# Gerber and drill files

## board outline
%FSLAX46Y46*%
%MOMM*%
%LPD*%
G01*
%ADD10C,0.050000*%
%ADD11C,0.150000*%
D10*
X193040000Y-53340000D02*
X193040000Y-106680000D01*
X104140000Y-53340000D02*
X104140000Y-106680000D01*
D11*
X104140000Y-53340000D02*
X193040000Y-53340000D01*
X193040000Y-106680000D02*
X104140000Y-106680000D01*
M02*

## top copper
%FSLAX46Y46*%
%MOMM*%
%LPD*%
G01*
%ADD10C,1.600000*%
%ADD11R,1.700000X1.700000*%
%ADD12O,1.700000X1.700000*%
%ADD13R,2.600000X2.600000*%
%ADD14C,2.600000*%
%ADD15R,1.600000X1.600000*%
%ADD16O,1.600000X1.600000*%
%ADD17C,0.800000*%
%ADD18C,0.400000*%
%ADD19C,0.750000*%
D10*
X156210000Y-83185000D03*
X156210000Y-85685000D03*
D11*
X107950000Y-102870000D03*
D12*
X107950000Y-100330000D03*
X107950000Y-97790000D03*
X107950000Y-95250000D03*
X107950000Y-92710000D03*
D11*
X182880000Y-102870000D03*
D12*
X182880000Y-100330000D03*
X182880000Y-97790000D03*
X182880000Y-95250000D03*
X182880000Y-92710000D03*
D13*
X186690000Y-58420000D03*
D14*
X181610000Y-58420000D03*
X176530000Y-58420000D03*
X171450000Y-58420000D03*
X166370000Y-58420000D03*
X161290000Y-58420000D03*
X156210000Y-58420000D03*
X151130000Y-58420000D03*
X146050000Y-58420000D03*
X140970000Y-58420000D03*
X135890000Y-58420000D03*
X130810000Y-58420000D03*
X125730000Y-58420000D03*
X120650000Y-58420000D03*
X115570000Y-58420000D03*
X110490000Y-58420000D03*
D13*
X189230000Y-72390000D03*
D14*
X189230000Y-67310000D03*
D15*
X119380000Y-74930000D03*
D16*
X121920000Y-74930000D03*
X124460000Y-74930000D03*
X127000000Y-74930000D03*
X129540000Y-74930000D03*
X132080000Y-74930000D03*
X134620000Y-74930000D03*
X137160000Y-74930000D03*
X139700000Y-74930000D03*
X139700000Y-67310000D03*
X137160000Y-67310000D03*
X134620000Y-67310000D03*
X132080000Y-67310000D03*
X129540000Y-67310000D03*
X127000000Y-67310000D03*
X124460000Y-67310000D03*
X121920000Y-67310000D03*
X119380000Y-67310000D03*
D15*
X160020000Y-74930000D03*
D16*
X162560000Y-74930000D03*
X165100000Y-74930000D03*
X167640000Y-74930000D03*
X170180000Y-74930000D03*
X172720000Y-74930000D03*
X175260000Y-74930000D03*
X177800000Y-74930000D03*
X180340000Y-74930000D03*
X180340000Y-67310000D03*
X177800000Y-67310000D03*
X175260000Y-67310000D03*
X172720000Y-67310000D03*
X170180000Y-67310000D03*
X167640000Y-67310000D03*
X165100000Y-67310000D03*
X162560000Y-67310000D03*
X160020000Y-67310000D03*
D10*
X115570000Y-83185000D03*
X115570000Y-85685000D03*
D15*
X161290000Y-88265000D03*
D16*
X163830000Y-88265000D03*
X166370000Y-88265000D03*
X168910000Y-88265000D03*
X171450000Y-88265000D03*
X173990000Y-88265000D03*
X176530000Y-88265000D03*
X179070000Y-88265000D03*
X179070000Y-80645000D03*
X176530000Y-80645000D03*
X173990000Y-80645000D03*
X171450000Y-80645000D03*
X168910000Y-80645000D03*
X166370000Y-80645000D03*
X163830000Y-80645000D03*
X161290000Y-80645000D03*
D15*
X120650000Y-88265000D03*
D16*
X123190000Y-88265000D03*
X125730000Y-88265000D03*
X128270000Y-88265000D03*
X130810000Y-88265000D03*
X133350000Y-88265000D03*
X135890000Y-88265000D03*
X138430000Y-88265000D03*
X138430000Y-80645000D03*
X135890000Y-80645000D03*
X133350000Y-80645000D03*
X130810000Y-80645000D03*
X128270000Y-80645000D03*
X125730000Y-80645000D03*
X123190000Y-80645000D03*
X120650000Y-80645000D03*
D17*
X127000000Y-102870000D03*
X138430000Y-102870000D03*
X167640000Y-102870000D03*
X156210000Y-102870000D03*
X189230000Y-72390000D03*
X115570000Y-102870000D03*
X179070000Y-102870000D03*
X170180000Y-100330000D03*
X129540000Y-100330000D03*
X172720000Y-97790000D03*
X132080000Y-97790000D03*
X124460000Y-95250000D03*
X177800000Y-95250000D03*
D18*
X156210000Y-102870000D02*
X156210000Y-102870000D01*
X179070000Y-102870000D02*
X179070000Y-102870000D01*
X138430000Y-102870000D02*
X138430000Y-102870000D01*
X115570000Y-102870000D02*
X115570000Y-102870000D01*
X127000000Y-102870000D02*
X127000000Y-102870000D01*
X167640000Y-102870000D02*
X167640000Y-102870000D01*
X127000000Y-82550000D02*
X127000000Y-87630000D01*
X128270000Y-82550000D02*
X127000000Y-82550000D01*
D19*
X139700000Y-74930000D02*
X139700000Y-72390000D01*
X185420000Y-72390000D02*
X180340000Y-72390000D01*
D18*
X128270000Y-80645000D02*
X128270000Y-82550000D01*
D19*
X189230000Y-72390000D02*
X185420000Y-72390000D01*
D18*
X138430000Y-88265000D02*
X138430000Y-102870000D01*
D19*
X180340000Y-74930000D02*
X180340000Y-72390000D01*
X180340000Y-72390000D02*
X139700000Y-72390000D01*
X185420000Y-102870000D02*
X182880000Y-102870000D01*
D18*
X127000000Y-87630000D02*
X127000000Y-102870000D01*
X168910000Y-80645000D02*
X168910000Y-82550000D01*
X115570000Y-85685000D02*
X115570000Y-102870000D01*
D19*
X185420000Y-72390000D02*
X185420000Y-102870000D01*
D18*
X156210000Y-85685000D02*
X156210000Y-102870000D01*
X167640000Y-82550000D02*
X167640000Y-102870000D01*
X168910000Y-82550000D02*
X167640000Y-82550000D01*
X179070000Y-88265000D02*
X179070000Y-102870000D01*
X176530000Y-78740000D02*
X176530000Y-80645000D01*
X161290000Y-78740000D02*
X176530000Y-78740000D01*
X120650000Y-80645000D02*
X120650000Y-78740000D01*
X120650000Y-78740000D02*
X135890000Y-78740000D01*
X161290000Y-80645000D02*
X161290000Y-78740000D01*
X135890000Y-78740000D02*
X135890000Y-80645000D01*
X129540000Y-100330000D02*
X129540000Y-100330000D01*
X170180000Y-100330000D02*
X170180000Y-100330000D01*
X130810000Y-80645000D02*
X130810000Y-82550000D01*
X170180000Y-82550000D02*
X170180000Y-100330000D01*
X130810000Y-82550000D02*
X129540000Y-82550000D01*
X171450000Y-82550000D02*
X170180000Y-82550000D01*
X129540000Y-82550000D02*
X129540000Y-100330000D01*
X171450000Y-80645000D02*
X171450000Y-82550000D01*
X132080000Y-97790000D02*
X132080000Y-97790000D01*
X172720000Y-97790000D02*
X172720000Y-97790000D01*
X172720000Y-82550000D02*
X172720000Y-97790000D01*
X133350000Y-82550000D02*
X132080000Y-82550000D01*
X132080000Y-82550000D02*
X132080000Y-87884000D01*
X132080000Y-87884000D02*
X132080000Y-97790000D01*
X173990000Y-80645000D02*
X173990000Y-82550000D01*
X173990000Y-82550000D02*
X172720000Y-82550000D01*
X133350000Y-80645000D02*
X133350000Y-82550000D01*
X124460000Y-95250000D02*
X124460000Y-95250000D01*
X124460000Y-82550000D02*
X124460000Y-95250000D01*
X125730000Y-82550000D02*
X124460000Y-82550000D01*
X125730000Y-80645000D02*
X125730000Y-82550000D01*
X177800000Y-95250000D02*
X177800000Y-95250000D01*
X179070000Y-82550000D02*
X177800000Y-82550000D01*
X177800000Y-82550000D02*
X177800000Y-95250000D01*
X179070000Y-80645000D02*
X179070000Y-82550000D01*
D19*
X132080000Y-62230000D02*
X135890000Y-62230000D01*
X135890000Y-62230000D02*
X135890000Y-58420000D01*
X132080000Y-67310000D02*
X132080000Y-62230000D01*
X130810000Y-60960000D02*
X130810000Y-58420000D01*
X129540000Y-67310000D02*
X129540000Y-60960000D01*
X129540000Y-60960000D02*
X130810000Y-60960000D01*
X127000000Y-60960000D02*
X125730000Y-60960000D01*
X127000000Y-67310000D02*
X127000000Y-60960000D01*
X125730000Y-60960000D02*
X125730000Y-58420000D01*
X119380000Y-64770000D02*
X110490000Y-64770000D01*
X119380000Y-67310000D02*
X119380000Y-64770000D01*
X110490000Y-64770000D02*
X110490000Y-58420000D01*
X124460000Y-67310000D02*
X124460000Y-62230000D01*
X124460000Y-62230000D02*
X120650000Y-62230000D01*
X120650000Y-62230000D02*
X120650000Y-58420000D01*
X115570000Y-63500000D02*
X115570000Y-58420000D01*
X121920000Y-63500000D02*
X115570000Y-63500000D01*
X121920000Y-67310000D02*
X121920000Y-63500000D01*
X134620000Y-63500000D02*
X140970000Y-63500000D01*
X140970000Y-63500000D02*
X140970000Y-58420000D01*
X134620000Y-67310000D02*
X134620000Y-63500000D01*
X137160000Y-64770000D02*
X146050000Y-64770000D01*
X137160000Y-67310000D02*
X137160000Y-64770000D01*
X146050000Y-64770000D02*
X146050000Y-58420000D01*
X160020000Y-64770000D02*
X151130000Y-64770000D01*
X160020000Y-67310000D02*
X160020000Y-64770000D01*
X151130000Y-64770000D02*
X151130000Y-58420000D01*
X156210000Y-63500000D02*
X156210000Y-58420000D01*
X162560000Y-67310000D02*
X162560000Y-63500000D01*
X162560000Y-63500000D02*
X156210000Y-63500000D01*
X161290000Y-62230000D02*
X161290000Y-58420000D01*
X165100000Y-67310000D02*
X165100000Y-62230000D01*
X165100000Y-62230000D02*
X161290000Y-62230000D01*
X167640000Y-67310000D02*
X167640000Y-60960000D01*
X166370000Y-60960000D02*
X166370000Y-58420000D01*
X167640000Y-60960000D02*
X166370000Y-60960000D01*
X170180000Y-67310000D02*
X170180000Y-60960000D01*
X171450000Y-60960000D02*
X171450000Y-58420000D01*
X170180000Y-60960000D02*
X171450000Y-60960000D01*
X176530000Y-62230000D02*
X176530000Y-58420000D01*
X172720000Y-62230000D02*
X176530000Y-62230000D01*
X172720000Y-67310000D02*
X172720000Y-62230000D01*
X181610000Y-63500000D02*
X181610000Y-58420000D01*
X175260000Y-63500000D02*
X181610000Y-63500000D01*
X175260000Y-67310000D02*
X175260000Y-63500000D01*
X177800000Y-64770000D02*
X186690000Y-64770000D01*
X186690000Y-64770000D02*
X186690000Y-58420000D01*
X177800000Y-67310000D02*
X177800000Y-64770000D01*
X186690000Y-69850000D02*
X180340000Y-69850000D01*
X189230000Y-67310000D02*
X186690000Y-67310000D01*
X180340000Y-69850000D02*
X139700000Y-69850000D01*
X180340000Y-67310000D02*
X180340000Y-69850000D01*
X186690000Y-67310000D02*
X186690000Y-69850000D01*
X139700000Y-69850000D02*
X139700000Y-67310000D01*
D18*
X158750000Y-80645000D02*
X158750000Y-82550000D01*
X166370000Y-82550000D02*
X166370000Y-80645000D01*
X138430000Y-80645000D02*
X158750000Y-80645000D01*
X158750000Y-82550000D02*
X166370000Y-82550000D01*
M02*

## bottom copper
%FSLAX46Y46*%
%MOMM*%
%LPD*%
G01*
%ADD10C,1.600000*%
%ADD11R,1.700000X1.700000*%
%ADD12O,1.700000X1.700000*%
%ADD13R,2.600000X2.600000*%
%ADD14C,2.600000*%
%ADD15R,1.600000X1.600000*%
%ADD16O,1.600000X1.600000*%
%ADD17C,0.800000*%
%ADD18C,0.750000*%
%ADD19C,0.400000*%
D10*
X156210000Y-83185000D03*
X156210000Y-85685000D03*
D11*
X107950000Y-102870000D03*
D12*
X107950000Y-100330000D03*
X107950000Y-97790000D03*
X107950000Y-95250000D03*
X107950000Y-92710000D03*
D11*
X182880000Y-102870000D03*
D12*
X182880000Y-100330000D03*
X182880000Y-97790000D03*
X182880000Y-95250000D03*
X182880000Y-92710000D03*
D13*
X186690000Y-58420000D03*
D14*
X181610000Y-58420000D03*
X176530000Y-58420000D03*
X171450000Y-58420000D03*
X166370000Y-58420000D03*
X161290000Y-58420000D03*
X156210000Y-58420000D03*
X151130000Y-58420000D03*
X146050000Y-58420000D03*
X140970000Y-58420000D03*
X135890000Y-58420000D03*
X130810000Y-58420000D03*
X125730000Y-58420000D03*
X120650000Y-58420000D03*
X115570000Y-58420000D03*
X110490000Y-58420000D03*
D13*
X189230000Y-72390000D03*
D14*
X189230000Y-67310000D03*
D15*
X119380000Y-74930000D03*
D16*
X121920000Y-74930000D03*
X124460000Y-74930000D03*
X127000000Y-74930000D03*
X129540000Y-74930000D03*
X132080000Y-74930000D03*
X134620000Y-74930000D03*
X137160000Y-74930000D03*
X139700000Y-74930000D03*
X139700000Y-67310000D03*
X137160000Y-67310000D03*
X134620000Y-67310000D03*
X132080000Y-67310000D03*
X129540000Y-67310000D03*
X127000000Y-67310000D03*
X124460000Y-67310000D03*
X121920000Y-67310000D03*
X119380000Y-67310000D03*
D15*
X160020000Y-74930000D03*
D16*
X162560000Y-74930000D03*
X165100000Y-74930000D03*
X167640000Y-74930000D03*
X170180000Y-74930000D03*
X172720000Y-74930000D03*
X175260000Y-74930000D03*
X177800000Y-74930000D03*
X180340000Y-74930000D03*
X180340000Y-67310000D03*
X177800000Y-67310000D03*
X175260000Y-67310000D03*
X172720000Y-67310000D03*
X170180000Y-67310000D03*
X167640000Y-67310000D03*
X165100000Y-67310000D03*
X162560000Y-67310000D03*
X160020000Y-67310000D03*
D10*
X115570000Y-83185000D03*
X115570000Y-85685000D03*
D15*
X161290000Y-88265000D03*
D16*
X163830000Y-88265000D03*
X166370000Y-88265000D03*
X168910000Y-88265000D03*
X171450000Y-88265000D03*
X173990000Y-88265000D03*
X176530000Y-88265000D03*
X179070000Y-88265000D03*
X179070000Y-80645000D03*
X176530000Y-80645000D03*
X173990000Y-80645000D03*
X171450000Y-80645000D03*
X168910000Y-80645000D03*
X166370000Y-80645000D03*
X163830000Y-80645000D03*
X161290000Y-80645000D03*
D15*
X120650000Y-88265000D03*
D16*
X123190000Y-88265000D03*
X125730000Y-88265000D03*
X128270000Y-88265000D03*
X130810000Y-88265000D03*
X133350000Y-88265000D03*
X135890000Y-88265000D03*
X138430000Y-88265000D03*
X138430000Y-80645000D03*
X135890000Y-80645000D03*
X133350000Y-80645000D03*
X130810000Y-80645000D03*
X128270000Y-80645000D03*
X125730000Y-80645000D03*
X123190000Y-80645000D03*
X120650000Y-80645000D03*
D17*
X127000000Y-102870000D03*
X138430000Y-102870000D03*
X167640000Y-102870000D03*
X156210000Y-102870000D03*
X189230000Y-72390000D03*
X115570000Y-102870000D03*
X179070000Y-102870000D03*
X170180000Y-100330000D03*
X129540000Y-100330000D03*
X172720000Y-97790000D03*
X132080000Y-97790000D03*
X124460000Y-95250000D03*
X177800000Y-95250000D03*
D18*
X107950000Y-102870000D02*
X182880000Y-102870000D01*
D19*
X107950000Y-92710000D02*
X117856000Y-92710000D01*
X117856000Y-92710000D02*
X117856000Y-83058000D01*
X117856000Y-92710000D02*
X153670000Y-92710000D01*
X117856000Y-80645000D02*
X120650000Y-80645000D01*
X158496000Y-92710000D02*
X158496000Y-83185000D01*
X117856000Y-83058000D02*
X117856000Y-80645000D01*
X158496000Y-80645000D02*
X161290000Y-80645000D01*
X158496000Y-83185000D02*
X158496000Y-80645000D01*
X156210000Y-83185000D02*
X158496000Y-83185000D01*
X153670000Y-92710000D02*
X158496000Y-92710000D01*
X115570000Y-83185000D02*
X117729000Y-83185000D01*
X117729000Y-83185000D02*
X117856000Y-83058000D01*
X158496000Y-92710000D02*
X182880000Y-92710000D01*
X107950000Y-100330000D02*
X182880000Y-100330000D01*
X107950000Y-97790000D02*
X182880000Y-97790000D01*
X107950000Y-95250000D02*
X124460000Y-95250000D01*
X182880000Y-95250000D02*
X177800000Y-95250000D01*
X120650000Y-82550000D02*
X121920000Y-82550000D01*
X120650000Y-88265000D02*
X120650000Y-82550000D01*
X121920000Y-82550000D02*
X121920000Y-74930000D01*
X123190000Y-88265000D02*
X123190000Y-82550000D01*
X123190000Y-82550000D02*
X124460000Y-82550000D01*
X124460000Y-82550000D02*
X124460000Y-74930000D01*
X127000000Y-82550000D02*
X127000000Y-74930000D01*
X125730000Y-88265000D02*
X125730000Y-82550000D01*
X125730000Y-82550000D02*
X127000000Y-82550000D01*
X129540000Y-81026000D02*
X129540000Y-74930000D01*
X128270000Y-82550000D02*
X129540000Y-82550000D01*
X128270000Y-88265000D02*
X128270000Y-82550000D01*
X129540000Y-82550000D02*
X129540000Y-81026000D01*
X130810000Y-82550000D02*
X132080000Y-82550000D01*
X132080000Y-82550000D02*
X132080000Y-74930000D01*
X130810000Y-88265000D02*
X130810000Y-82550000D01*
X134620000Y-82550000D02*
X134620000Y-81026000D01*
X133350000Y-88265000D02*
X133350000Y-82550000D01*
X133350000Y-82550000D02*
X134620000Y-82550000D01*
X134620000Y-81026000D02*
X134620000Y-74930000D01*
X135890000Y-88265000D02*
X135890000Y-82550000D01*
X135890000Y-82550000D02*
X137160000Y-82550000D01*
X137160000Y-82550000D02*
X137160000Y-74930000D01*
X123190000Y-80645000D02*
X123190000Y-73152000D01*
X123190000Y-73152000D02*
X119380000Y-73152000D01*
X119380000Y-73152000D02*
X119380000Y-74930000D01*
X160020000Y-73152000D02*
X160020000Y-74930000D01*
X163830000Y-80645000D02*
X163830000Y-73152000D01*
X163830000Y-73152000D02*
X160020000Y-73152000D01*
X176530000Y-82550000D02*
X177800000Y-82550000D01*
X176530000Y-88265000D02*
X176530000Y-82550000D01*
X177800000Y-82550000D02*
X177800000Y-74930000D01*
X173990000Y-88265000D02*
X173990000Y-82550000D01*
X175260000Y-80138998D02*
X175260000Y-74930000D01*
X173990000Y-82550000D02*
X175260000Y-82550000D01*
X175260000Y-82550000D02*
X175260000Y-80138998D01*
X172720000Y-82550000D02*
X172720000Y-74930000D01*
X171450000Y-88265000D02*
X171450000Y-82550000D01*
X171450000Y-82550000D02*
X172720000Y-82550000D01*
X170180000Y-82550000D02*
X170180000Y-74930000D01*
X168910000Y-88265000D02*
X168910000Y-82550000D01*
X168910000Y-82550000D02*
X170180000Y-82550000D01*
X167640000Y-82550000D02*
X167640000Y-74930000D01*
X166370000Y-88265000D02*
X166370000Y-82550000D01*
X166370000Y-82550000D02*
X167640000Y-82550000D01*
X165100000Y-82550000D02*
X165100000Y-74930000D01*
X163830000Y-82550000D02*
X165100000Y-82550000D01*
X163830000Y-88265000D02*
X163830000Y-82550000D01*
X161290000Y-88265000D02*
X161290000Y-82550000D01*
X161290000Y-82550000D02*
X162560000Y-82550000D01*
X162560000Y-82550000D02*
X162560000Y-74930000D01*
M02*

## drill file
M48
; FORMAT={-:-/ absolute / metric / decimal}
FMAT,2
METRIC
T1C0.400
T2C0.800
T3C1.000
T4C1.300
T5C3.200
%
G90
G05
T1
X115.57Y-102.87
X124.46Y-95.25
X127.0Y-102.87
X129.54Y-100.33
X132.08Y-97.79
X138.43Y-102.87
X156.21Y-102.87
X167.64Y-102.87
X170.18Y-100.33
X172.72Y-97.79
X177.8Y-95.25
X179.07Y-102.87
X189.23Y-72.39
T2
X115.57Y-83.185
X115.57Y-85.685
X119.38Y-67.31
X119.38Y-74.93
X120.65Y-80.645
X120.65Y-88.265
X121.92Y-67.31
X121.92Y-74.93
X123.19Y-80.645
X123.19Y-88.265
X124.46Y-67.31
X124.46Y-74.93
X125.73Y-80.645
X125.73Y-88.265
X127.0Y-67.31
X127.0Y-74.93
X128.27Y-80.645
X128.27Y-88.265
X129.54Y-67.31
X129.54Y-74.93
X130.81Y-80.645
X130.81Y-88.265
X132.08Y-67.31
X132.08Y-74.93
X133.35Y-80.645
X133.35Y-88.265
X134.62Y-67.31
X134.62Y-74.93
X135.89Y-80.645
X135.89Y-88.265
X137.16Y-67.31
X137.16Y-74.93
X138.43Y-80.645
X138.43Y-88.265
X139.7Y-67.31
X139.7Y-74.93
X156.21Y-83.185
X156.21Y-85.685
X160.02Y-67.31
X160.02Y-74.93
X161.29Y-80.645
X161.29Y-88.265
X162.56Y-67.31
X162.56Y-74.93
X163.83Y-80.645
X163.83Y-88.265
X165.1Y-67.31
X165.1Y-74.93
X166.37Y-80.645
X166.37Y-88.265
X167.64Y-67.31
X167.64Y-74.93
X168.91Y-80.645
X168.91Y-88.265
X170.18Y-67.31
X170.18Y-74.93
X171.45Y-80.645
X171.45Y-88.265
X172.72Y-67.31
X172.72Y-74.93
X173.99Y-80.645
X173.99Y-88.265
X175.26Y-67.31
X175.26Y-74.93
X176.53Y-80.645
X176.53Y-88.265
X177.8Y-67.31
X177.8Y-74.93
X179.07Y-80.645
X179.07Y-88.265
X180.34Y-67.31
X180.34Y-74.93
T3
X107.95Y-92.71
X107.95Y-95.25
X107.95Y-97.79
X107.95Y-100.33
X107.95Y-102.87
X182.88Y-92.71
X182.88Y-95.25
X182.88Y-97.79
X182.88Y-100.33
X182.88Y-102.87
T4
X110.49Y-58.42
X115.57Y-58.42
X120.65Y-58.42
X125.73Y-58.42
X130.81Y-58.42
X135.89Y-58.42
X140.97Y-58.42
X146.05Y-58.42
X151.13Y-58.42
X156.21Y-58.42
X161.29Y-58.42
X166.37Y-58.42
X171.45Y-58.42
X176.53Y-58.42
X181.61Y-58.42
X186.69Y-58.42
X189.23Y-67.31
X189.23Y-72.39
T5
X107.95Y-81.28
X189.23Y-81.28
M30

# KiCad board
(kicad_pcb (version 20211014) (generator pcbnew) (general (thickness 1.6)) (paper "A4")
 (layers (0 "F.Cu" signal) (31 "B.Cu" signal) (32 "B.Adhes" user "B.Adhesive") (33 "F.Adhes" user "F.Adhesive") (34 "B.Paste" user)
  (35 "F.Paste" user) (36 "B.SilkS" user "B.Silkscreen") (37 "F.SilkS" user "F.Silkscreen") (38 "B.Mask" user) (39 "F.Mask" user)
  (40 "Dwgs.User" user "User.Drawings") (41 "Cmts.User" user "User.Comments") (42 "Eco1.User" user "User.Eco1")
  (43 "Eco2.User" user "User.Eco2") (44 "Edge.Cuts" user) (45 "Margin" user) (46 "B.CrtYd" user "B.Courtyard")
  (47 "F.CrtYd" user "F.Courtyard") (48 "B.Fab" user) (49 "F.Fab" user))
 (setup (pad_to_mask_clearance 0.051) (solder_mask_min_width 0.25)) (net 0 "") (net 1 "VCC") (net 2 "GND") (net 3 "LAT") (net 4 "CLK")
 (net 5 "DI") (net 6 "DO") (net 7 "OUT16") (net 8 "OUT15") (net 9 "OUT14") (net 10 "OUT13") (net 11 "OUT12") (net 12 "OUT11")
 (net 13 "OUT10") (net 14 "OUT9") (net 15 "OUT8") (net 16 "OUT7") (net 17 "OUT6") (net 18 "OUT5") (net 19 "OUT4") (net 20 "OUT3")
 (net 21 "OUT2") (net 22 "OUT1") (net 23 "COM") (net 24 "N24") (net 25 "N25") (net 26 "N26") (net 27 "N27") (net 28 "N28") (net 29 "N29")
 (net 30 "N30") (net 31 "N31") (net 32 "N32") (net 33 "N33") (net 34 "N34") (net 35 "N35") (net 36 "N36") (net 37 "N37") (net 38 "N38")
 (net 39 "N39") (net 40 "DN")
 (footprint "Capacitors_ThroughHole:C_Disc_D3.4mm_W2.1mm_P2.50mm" (layer "F.Cu") (at 156.21 83.185 -90)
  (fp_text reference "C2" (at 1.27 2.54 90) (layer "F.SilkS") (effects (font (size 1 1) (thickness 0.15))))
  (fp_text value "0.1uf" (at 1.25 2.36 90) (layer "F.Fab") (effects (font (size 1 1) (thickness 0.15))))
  (pad "1" thru_hole circle locked (at 0 0 270) (size 1.6 1.6) (drill 0.8) (layers *.Cu *.Mask) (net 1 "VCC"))
  (pad "2" thru_hole circle locked (at 2.5 0 270) (size 1.6 1.6) (drill 0.8) (layers *.Cu *.Mask) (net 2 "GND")))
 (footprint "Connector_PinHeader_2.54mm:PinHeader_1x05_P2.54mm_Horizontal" (layer "F.Cu") (at 107.95 102.87 180)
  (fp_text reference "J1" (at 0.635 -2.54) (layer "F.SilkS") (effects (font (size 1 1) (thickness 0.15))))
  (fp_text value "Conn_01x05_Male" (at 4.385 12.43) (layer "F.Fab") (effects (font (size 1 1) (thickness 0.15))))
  (pad "1" thru_hole rect locked (at 0 0 180) (size 1.7 1.7) (drill 1) (layers *.Cu *.Mask) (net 2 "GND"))
  (pad "2" thru_hole oval locked (at 0 2.54 180) (size 1.7 1.7) (drill 1) (layers *.Cu *.Mask) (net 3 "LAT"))
  (pad "3" thru_hole oval locked (at 0 5.08 180) (size 1.7 1.7) (drill 1) (layers *.Cu *.Mask) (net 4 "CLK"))
  (pad "4" thru_hole oval locked (at 0 7.62 180) (size 1.7 1.7) (drill 1) (layers *.Cu *.Mask) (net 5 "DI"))
  (pad "5" thru_hole oval locked (at 0 10.16 180) (size 1.7 1.7) (drill 1) (layers *.Cu *.Mask) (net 1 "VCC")))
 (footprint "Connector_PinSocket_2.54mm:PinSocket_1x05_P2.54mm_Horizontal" (layer "F.Cu") (at 182.88 102.87 180)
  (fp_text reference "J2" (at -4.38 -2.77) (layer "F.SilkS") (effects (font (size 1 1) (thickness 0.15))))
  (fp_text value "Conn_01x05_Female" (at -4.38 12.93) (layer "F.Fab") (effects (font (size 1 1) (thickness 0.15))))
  (pad "1" thru_hole rect locked (at 0 0 180) (size 1.7 1.7) (drill 1) (layers *.Cu *.Mask) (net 2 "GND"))
  (pad "2" thru_hole oval locked (at 0 2.54 180) (size 1.7 1.7) (drill 1) (layers *.Cu *.Mask) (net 3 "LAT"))
  (pad "3" thru_hole oval locked (at 0 5.08 180) (size 1.7 1.7) (drill 1) (layers *.Cu *.Mask) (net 4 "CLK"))
  (pad "4" thru_hole oval locked (at 0 7.62 180) (size 1.7 1.7) (drill 1) (layers *.Cu *.Mask) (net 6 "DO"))
  (pad "5" thru_hole oval locked (at 0 10.16 180) (size 1.7 1.7) (drill 1) (layers *.Cu *.Mask) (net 1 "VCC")))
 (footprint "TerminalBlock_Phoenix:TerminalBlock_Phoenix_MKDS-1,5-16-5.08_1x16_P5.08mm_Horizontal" (layer "F.Cu") (at 186.69 58.42 180)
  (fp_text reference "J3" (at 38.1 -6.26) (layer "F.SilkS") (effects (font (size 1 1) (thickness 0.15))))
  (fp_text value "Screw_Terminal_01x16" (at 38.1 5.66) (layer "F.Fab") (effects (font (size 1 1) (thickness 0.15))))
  (pad "1" thru_hole rect locked (at 0 0 180) (size 2.6 2.6) (drill 1.3) (layers *.Cu *.Mask) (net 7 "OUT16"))
  (pad "2" thru_hole circle locked (at 5.08 0 180) (size 2.6 2.6) (drill 1.3) (layers *.Cu *.Mask) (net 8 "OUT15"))
  (pad "3" thru_hole circle locked (at 10.16 0 180) (size 2.6 2.6) (drill 1.3) (layers *.Cu *.Mask) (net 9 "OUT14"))
  (pad "4" thru_hole circle locked (at 15.24 0 180) (size 2.6 2.6) (drill 1.3) (layers *.Cu *.Mask) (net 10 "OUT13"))
  (pad "5" thru_hole circle locked (at 20.32 0 180) (size 2.6 2.6) (drill 1.3) (layers *.Cu *.Mask) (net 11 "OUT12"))
  (pad "6" thru_hole circle locked (at 25.4 0 180) (size 2.6 2.6) (drill 1.3) (layers *.Cu *.Mask) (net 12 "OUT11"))
  (pad "7" thru_hole circle locked (at 30.48 0 180) (size 2.6 2.6) (drill 1.3) (layers *.Cu *.Mask) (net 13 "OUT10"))
  (pad "8" thru_hole circle locked (at 35.56 0 180) (size 2.6 2.6) (drill 1.3) (layers *.Cu *.Mask) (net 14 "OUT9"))
  (pad "9" thru_hole circle locked (at 40.64 0 180) (size 2.6 2.6) (drill 1.3) (layers *.Cu *.Mask) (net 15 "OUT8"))
  (pad "10" thru_hole circle locked (at 45.72 0 180) (size 2.6 2.6) (drill 1.3) (layers *.Cu *.Mask) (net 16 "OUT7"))
  (pad "11" thru_hole circle locked (at 50.8 0 180) (size 2.6 2.6) (drill 1.3) (layers *.Cu *.Mask) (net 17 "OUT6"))
  (pad "12" thru_hole circle locked (at 55.88 0 180) (size 2.6 2.6) (drill 1.3) (layers *.Cu *.Mask) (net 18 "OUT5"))
  (pad "13" thru_hole circle locked (at 60.96 0 180) (size 2.6 2.6) (drill 1.3) (layers *.Cu *.Mask) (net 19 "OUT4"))
  (pad "14" thru_hole circle locked (at 66.04 0 180) (size 2.6 2.6) (drill 1.3) (layers *.Cu *.Mask) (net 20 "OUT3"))
  (pad "15" thru_hole circle locked (at 71.12 0 180) (size 2.6 2.6) (drill 1.3) (layers *.Cu *.Mask) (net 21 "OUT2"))
  (pad "16" thru_hole circle locked (at 76.2 0 180) (size 2.6 2.6) (drill 1.3) (layers *.Cu *.Mask) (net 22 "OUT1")))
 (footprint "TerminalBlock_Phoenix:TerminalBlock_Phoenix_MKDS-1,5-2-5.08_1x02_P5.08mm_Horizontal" (layer "F.Cu") (at 189.23 72.39 90)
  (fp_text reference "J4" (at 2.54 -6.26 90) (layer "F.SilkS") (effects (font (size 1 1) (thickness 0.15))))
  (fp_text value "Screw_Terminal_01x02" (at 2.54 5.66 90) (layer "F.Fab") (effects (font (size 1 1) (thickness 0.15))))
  (pad "1" thru_hole rect locked (at 0 0 90) (size 2.6 2.6) (drill 1.3) (layers *.Cu *.Mask) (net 2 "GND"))
  (pad "2" thru_hole circle locked (at 5.08 0 90) (size 2.6 2.6) (drill 1.3) (layers *.Cu *.Mask) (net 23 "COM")))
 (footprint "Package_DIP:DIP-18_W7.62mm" (layer "F.Cu") (at 119.38 74.93 90)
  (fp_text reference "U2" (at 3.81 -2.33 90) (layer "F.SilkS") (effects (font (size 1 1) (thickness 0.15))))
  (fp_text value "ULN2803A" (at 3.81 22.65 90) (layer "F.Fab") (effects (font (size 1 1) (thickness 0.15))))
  (pad "1" thru_hole rect locked (at 0 0 90) (size 1.6 1.6) (drill 0.8) (layers *.Cu *.Mask) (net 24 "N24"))
  (pad "2" thru_hole oval locked (at 0 2.54 90) (size 1.6 1.6) (drill 0.8) (layers *.Cu *.Mask) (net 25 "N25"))
  (pad "3" thru_hole oval locked (at 0 5.08 90) (size 1.6 1.6) (drill 0.8) (layers *.Cu *.Mask) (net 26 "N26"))
  (pad "4" thru_hole oval locked (at 0 7.62 90) (size 1.6 1.6) (drill 0.8) (layers *.Cu *.Mask) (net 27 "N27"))
  (pad "5" thru_hole oval locked (at 0 10.16 90) (size 1.6 1.6) (drill 0.8) (layers *.Cu *.Mask) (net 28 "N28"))
  (pad "6" thru_hole oval locked (at 0 12.7 90) (size 1.6 1.6) (drill 0.8) (layers *.Cu *.Mask) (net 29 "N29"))
  (pad "7" thru_hole oval locked (at 0 15.24 90) (size 1.6 1.6) (drill 0.8) (layers *.Cu *.Mask) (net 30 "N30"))
  (pad "8" thru_hole oval locked (at 0 17.78 90) (size 1.6 1.6) (drill 0.8) (layers *.Cu *.Mask) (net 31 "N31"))
  (pad "9" thru_hole oval locked (at 0 20.32 90) (size 1.6 1.6) (drill 0.8) (layers *.Cu *.Mask) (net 2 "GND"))
  (pad "10" thru_hole oval locked (at 7.62 20.32 90) (size 1.6 1.6) (drill 0.8) (layers *.Cu *.Mask) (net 23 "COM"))
  (pad "11" thru_hole oval locked (at 7.62 17.78 90) (size 1.6 1.6) (drill 0.8) (layers *.Cu *.Mask) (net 15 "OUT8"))
  (pad "12" thru_hole oval locked (at 7.62 15.24 90) (size 1.6 1.6) (drill 0.8) (layers *.Cu *.Mask) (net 16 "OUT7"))
  (pad "13" thru_hole oval locked (at 7.62 12.7 90) (size 1.6 1.6) (drill 0.8) (layers *.Cu *.Mask) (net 17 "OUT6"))
  (pad "14" thru_hole oval locked (at 7.62 10.16 90) (size 1.6 1.6) (drill 0.8) (layers *.Cu *.Mask) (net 18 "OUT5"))
  (pad "15" thru_hole oval locked (at 7.62 7.62 90) (size 1.6 1.6) (drill 0.8) (layers *.Cu *.Mask) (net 19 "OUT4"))
  (pad "16" thru_hole oval locked (at 7.62 5.08 90) (size 1.6 1.6) (drill 0.8) (layers *.Cu *.Mask) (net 20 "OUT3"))
  (pad "17" thru_hole oval locked (at 7.62 2.54 90) (size 1.6 1.6) (drill 0.8) (layers *.Cu *.Mask) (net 21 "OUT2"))
  (pad "18" thru_hole oval locked (at 7.62 0 90) (size 1.6 1.6) (drill 0.8) (layers *.Cu *.Mask) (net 22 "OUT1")))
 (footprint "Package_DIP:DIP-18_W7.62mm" (layer "F.Cu") (at 160.02 74.93 90)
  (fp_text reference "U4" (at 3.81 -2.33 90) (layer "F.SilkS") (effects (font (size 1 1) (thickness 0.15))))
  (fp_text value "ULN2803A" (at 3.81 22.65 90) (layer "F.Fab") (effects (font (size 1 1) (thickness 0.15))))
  (pad "1" thru_hole rect locked (at 0 0 90) (size 1.6 1.6) (drill 0.8) (layers *.Cu *.Mask) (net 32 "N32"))
  (pad "2" thru_hole oval locked (at 0 2.54 90) (size 1.6 1.6) (drill 0.8) (layers *.Cu *.Mask) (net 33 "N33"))
  (pad "3" thru_hole oval locked (at 0 5.08 90) (size 1.6 1.6) (drill 0.8) (layers *.Cu *.Mask) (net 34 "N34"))
  (pad "4" thru_hole oval locked (at 0 7.62 90) (size 1.6 1.6) (drill 0.8) (layers *.Cu *.Mask) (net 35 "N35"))
  (pad "5" thru_hole oval locked (at 0 10.16 90) (size 1.6 1.6) (drill 0.8) (layers *.Cu *.Mask) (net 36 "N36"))
  (pad "6" thru_hole oval locked (at 0 12.7 90) (size 1.6 1.6) (drill 0.8) (layers *.Cu *.Mask) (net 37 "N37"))
  (pad "7" thru_hole oval locked (at 0 15.24 90) (size 1.6 1.6) (drill 0.8) (layers *.Cu *.Mask) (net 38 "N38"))
  (pad "8" thru_hole oval locked (at 0 17.78 90) (size 1.6 1.6) (drill 0.8) (layers *.Cu *.Mask) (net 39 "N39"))
  (pad "9" thru_hole oval locked (at 0 20.32 90) (size 1.6 1.6) (drill 0.8) (layers *.Cu *.Mask) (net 2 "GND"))
  (pad "10" thru_hole oval locked (at 7.62 20.32 90) (size 1.6 1.6) (drill 0.8) (layers *.Cu *.Mask) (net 23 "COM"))
  (pad "11" thru_hole oval locked (at 7.62 17.78 90) (size 1.6 1.6) (drill 0.8) (layers *.Cu *.Mask) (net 7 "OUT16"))
  (pad "12" thru_hole oval locked (at 7.62 15.24 90) (size 1.6 1.6) (drill 0.8) (layers *.Cu *.Mask) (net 8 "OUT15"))
  (pad "13" thru_hole oval locked (at 7.62 12.7 90) (size 1.6 1.6) (drill 0.8) (layers *.Cu *.Mask) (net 9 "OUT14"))
  (pad "14" thru_hole oval locked (at 7.62 10.16 90) (size 1.6 1.6) (drill 0.8) (layers *.Cu *.Mask) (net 10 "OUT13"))
  (pad "15" thru_hole oval locked (at 7.62 7.62 90) (size 1.6 1.6) (drill 0.8) (layers *.Cu *.Mask) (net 11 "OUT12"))
  (pad "16" thru_hole oval locked (at 7.62 5.08 90) (size 1.6 1.6) (drill 0.8) (layers *.Cu *.Mask) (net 12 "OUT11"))
  (pad "17" thru_hole oval locked (at 7.62 2.54 90) (size 1.6 1.6) (drill 0.8) (layers *.Cu *.Mask) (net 13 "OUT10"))
  (pad "18" thru_hole oval locked (at 7.62 0 90) (size 1.6 1.6) (drill 0.8) (layers *.Cu *.Mask) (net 14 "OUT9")))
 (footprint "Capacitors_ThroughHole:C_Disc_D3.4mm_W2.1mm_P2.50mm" (layer "F.Cu") (at 115.57 83.185 -90)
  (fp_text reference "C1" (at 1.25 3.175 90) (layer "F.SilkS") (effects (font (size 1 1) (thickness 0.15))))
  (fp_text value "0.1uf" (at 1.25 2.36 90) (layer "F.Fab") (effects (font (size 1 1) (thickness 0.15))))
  (pad "1" thru_hole circle locked (at 0 0 270) (size 1.6 1.6) (drill 0.8) (layers *.Cu *.Mask) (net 1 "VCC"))
  (pad "2" thru_hole circle locked (at 2.5 0 270) (size 1.6 1.6) (drill 0.8) (layers *.Cu *.Mask) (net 2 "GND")))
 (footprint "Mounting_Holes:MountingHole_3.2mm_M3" (layer "F.Cu") (at 107.95 81.28)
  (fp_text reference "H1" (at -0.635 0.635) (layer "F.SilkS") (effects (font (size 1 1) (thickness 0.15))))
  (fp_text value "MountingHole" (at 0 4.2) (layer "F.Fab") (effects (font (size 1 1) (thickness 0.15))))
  (pad "" np_thru_hole circle locked (at 0 0) (size 3.2 3.2) (drill 3.2) (layers *.Cu *.Mask)))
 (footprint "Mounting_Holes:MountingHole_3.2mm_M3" (layer "F.Cu") (at 189.23 81.28)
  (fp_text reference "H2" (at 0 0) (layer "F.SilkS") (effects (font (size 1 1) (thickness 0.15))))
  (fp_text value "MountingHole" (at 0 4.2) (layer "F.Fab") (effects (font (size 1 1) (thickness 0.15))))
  (pad "" np_thru_hole circle locked (at 0 0) (size 3.2 3.2) (drill 3.2) (layers *.Cu *.Mask)))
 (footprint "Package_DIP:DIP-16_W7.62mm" (layer "F.Cu") (at 161.29 88.265 90)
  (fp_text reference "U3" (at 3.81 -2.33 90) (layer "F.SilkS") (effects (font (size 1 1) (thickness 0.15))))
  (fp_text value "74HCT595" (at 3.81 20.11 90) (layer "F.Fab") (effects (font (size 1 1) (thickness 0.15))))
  (pad "1" thru_hole rect locked (at 0 0 90) (size 1.6 1.6) (drill 0.8) (layers *.Cu *.Mask) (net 33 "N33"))
  (pad "2" thru_hole oval locked (at 0 2.54 90) (size 1.6 1.6) (drill 0.8) (layers *.Cu *.Mask) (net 34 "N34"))
  (pad "3" thru_hole oval locked (at 0 5.08 90) (size 1.6 1.6) (drill 0.8) (layers *.Cu *.Mask) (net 35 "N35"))
  (pad "4" thru_hole oval locked (at 0 7.62 90) (size 1.6 1.6) (drill 0.8) (layers *.Cu *.Mask) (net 36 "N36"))
  (pad "5" thru_hole oval locked (at 0 10.16 90) (size 1.6 1.6) (drill 0.8) (layers *.Cu *.Mask) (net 37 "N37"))
  (pad "6" thru_hole oval locked (at 0 12.7 90) (size 1.6 1.6) (drill 0.8) (layers *.Cu *.Mask) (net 38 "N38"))
  (pad "7" thru_hole oval locked (at 0 15.24 90) (size 1.6 1.6) (drill 0.8) (layers *.Cu *.Mask) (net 39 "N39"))
  (pad "8" thru_hole oval locked (at 0 17.78 90) (size 1.6 1.6) (drill 0.8) (layers *.Cu *.Mask) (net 2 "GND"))
  (pad "9" thru_hole oval locked (at 7.62 17.78 90) (size 1.6 1.6) (drill 0.8) (layers *.Cu *.Mask) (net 6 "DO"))
  (pad "10" thru_hole oval locked (at 7.62 15.24 90) (size 1.6 1.6) (drill 0.8) (layers *.Cu *.Mask) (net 1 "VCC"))
  (pad "11" thru_hole oval locked (at 7.62 12.7 90) (size 1.6 1.6) (drill 0.8) (layers *.Cu *.Mask) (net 4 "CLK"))
  (pad "12" thru_hole oval locked (at 7.62 10.16 90) (size 1.6 1.6) (drill 0.8) (layers *.Cu *.Mask) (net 3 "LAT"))
  (pad "13" thru_hole oval locked (at 7.62 7.62 90) (size 1.6 1.6) (drill 0.8) (layers *.Cu *.Mask) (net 2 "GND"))
  (pad "14" thru_hole oval locked (at 7.62 5.08 90) (size 1.6 1.6) (drill 0.8) (layers *.Cu *.Mask) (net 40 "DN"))
  (pad "15" thru_hole oval locked (at 7.62 2.54 90) (size 1.6 1.6) (drill 0.8) (layers *.Cu *.Mask) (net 32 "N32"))
  (pad "16" thru_hole oval locked (at 7.62 0 90) (size 1.6 1.6) (drill 0.8) (layers *.Cu *.Mask) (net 1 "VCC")))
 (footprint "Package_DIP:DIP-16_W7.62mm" (layer "F.Cu") (at 120.65 88.265 90)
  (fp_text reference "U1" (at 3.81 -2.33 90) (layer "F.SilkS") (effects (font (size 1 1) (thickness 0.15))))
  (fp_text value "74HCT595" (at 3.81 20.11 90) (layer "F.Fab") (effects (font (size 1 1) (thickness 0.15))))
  (pad "1" thru_hole rect locked (at 0 0 90) (size 1.6 1.6) (drill 0.8) (layers *.Cu *.Mask) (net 25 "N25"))
  (pad "2" thru_hole oval locked (at 0 2.54 90) (size 1.6 1.6) (drill 0.8) (layers *.Cu *.Mask) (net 26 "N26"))
  (pad "3" thru_hole oval locked (at 0 5.08 90) (size 1.6 1.6) (drill 0.8) (layers *.Cu *.Mask) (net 27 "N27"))
  (pad "4" thru_hole oval locked (at 0 7.62 90) (size 1.6 1.6) (drill 0.8) (layers *.Cu *.Mask) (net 28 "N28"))
  (pad "5" thru_hole oval locked (at 0 10.16 90) (size 1.6 1.6) (drill 0.8) (layers *.Cu *.Mask) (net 29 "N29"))
  (pad "6" thru_hole oval locked (at 0 12.7 90) (size 1.6 1.6) (drill 0.8) (layers *.Cu *.Mask) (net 30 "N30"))
  (pad "7" thru_hole oval locked (at 0 15.24 90) (size 1.6 1.6) (drill 0.8) (layers *.Cu *.Mask) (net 31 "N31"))
  (pad "8" thru_hole oval locked (at 0 17.78 90) (size 1.6 1.6) (drill 0.8) (layers *.Cu *.Mask) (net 2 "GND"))
  (pad "9" thru_hole oval locked (at 7.62 17.78 90) (size 1.6 1.6) (drill 0.8) (layers *.Cu *.Mask) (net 40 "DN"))
  (pad "10" thru_hole oval locked (at 7.62 15.24 90) (size 1.6 1.6) (drill 0.8) (layers *.Cu *.Mask) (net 1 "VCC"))
  (pad "11" thru_hole oval locked (at 7.62 12.7 90) (size 1.6 1.6) (drill 0.8) (layers *.Cu *.Mask) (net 4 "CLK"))
  (pad "12" thru_hole oval locked (at 7.62 10.16 90) (size 1.6 1.6) (drill 0.8) (layers *.Cu *.Mask) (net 3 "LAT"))
  (pad "13" thru_hole oval locked (at 7.62 7.62 90) (size 1.6 1.6) (drill 0.8) (layers *.Cu *.Mask) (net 2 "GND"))
  (pad "14" thru_hole oval locked (at 7.62 5.08 90) (size 1.6 1.6) (drill 0.8) (layers *.Cu *.Mask) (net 5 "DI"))
  (pad "15" thru_hole oval locked (at 7.62 2.54 90) (size 1.6 1.6) (drill 0.8) (layers *.Cu *.Mask) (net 24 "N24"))
  (pad "16" thru_hole oval locked (at 7.62 0 90) (size 1.6 1.6) (drill 0.8) (layers *.Cu *.Mask) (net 1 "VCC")))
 (gr_line (start 193.04 53.34) (end 193.04 106.68) (layer "Edge.Cuts") (width 0.05))
 (gr_line (start 104.14 53.34) (end 104.14 106.68) (layer "Edge.Cuts") (width 0.05))
 (gr_line (start 104.14 53.34) (end 193.04 53.34) (layer "Edge.Cuts") (width 0.15))
 (gr_line (start 193.04 106.68) (end 104.14 106.68) (layer "Edge.Cuts") (width 0.15))
 (segment (start 156.21 102.87) (end 156.21 102.87) (width 0.4) (layer "F.Cu") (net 2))
 (segment (start 179.07 102.87) (end 179.07 102.87) (width 0.4) (layer "F.Cu") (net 2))
 (segment (start 138.43 102.87) (end 138.43 102.87) (width 0.4) (layer "F.Cu") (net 2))
 (segment (start 115.57 102.87) (end 115.57 102.87) (width 0.4) (layer "F.Cu") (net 2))
 (segment (start 127 102.87) (end 127 102.87) (width 0.4) (layer "F.Cu") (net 2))
 (segment (start 167.64 102.87) (end 167.64 102.87) (width 0.4) (layer "F.Cu") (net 2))
 (segment (start 127 82.55) (end 127 87.63) (width 0.4) (layer "F.Cu") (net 2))
 (segment (start 128.27 82.55) (end 127 82.55) (width 0.4) (layer "F.Cu") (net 2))
 (segment (start 139.7 74.93) (end 139.7 72.39) (width 0.75) (layer "F.Cu") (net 2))
 (segment (start 185.42 72.39) (end 180.34 72.39) (width 0.75) (layer "F.Cu") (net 2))
 (segment (start 128.27 80.645) (end 128.27 82.55) (width 0.4) (layer "F.Cu") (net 2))
 (segment (start 189.23 72.39) (end 185.42 72.39) (width 0.75) (layer "F.Cu") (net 2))
 (segment (start 138.43 88.265) (end 138.43 102.87) (width 0.4) (layer "F.Cu") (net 2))
 (segment (start 180.34 74.93) (end 180.34 72.39) (width 0.75) (layer "F.Cu") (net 2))
 (segment (start 180.34 72.39) (end 139.7 72.39) (width 0.75) (layer "F.Cu") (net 2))
 (segment (start 185.42 102.87) (end 182.88 102.87) (width 0.75) (layer "F.Cu") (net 2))
 (segment (start 127 87.63) (end 127 102.87) (width 0.4) (layer "F.Cu") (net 2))
 (segment (start 168.91 80.645) (end 168.91 82.55) (width 0.4) (layer "F.Cu") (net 2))
 (segment (start 115.57 85.685) (end 115.57 102.87) (width 0.4) (layer "F.Cu") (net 2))
 (segment (start 185.42 72.39) (end 185.42 102.87) (width 0.75) (layer "F.Cu") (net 2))
 (segment (start 156.21 85.685) (end 156.21 102.87) (width 0.4) (layer "F.Cu") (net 2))
 (segment (start 167.64 82.55) (end 167.64 102.87) (width 0.4) (layer "F.Cu") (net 2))
 (segment (start 168.91 82.55) (end 167.64 82.55) (width 0.4) (layer "F.Cu") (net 2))
 (segment (start 179.07 88.265) (end 179.07 102.87) (width 0.4) (layer "F.Cu") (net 2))
 (via (at 127 102.87) (size 0.8) (drill 0.4) (layers "F.Cu" "B.Cu") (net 2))
 (via (at 138.43 102.87) (size 0.8) (drill 0.4) (layers "F.Cu" "B.Cu") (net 2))
 (via (at 167.64 102.87) (size 0.8) (drill 0.4) (layers "F.Cu" "B.Cu") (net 2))
 (via (at 156.21 102.87) (size 0.8) (drill 0.4) (layers "F.Cu" "B.Cu") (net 2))
 (via (at 189.23 72.39) (size 0.8) (drill 0.4) (layers "F.Cu" "B.Cu") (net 2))
 (via (at 115.57 102.87) (size 0.8) (drill 0.4) (layers "F.Cu" "B.Cu") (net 2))
 (via (at 179.07 102.87) (size 0.8) (drill 0.4) (layers "F.Cu" "B.Cu") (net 2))
 (segment (start 107.95 102.87) (end 182.88 102.87) (width 0.75) (layer "B.Cu") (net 2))
 (segment (start 176.53 78.74) (end 176.53 80.645) (width 0.4) (layer "F.Cu") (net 1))
 (segment (start 161.29 78.74) (end 176.53 78.74) (width 0.4) (layer "F.Cu") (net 1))
 (segment (start 120.65 80.645) (end 120.65 78.74) (width 0.4) (layer "F.Cu") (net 1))
 (segment (start 120.65 78.74) (end 135.89 78.74) (width 0.4) (layer "F.Cu") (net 1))
 (segment (start 161.29 80.645) (end 161.29 78.74) (width 0.4) (layer "F.Cu") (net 1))
 (segment (start 135.89 78.74) (end 135.89 80.645) (width 0.4) (layer "F.Cu") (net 1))
 (segment (start 107.95 92.71) (end 117.856 92.71) (width 0.4) (layer "B.Cu") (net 1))
 (segment (start 117.856 92.71) (end 117.856 83.058) (width 0.4) (layer "B.Cu") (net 1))
 (segment (start 117.856 92.71) (end 153.67 92.71) (width 0.4) (layer "B.Cu") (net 1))
 (segment (start 117.856 80.645) (end 120.65 80.645) (width 0.4) (layer "B.Cu") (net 1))
 (segment (start 158.496 92.71) (end 158.496 83.185) (width 0.4) (layer "B.Cu") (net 1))
 (segment (start 117.856 83.058) (end 117.856 80.645) (width 0.4) (layer "B.Cu") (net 1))
 (segment (start 158.496 80.645) (end 161.29 80.645) (width 0.4) (layer "B.Cu") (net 1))
 (segment (start 158.496 83.185) (end 158.496 80.645) (width 0.4) (layer "B.Cu") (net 1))
 (segment (start 156.21 83.185) (end 158.496 83.185) (width 0.4) (layer "B.Cu") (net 1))
 (segment (start 153.67 92.71) (end 158.496 92.71) (width 0.4) (layer "B.Cu") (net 1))
 (segment (start 115.57 83.185) (end 117.729 83.185) (width 0.4) (layer "B.Cu") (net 1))
 (segment (start 117.729 83.185) (end 117.856 83.058) (width 0.4) (layer "B.Cu") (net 1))
 (segment (start 158.496 92.71) (end 182.88 92.71) (width 0.4) (layer "B.Cu") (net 1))
 (segment (start 129.54 100.33) (end 129.54 100.33) (width 0.4) (layer "F.Cu") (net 3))
 (segment (start 170.18 100.33) (end 170.18 100.33) (width 0.4) (layer "F.Cu") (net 3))
 (segment (start 130.81 80.645) (end 130.81 82.55) (width 0.4) (layer "F.Cu") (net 3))
 (segment (start 170.18 82.55) (end 170.18 100.33) (width 0.4) (layer "F.Cu") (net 3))
 (segment (start 130.81 82.55) (end 129.54 82.55) (width 0.4) (layer "F.Cu") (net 3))
 (segment (start 171.45 82.55) (end 170.18 82.55) (width 0.4) (layer "F.Cu") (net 3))
 (segment (start 129.54 82.55) (end 129.54 100.33) (width 0.4) (layer "F.Cu") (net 3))
 (segment (start 171.45 80.645) (end 171.45 82.55) (width 0.4) (layer "F.Cu") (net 3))
 (via (at 170.18 100.33) (size 0.8) (drill 0.4) (layers "F.Cu" "B.Cu") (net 3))
 (via (at 129.54 100.33) (size 0.8) (drill 0.4) (layers "F.Cu" "B.Cu") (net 3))
 (segment (start 107.95 100.33) (end 182.88 100.33) (width 0.4) (layer "B.Cu") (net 3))
 (segment (start 132.08 97.79) (end 132.08 97.79) (width 0.4) (layer "F.Cu") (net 4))
 (segment (start 172.72 97.79) (end 172.72 97.79) (width 0.4) (layer "F.Cu") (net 4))
 (segment (start 172.72 82.55) (end 172.72 97.79) (width 0.4) (layer "F.Cu") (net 4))
 (segment (start 133.35 82.55) (end 132.08 82.55) (width 0.4) (layer "F.Cu") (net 4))
 (segment (start 132.08 82.55) (end 132.08 87.884) (width 0.4) (layer "F.Cu") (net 4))
 (segment (start 132.08 87.884) (end 132.08 97.79) (width 0.4) (layer "F.Cu") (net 4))
 (segment (start 173.99 80.645) (end 173.99 82.55) (width 0.4) (layer "F.Cu") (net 4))
 (segment (start 173.99 82.55) (end 172.72 82.55) (width 0.4) (layer "F.Cu") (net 4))
 (segment (start 133.35 80.645) (end 133.35 82.55) (width 0.4) (layer "F.Cu") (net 4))
 (via (at 172.72 97.79) (size 0.8) (drill 0.4) (layers "F.Cu" "B.Cu") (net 4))
 (via (at 132.08 97.79) (size 0.8) (drill 0.4) (layers "F.Cu" "B.Cu") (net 4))
 (segment (start 107.95 97.79) (end 182.88 97.79) (width 0.4) (layer "B.Cu") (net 4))
 (segment (start 124.46 95.25) (end 124.46 95.25) (width 0.4) (layer "F.Cu") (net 5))
 (segment (start 124.46 82.55) (end 124.46 95.25) (width 0.4) (layer "F.Cu") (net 5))
 (segment (start 125.73 82.55) (end 124.46 82.55) (width 0.4) (layer "F.Cu") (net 5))
 (segment (start 125.73 80.645) (end 125.73 82.55) (width 0.4) (layer "F.Cu") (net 5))
 (via (at 124.46 95.25) (size 0.8) (drill 0.4) (layers "F.Cu" "B.Cu") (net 5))
 (segment (start 107.95 95.25) (end 124.46 95.25) (width 0.4) (layer "B.Cu") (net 5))
 (segment (start 177.8 95.25) (end 177.8 95.25) (width 0.4) (layer "F.Cu") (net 6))
 (segment (start 179.07 82.55) (end 177.8 82.55) (width 0.4) (layer "F.Cu") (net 6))
 (segment (start 177.8 82.55) (end 177.8 95.25) (width 0.4) (layer "F.Cu") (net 6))
 (segment (start 179.07 80.645) (end 179.07 82.55) (width 0.4) (layer "F.Cu") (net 6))
 (via (at 177.8 95.25) (size 0.8) (drill 0.4) (layers "F.Cu" "B.Cu") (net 6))
 (segment (start 182.88 95.25) (end 177.8 95.25) (width 0.4) (layer "B.Cu") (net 6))
 (segment (start 132.08 62.23) (end 135.89 62.23) (width 0.75) (layer "F.Cu") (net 17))
 (segment (start 135.89 62.23) (end 135.89 58.42) (width 0.75) (layer "F.Cu") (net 17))
 (segment (start 132.08 67.31) (end 132.08 62.23) (width 0.75) (layer "F.Cu") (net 17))
 (segment (start 130.81 60.96) (end 130.81 58.42) (width 0.75) (layer "F.Cu") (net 18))
 (segment (start 129.54 67.31) (end 129.54 60.96) (width 0.75) (layer "F.Cu") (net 18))
 (segment (start 129.54 60.96) (end 130.81 60.96) (width 0.75) (layer "F.Cu") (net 18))
 (segment (start 127 60.96) (end 125.73 60.96) (width 0.75) (layer "F.Cu") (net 19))
 (segment (start 127 67.31) (end 127 60.96) (width 0.75) (layer "F.Cu") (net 19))
 (segment (start 125.73 60.96) (end 125.73 58.42) (width 0.75) (layer "F.Cu") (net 19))
 (segment (start 119.38 64.77) (end 110.49 64.77) (width 0.75) (layer "F.Cu") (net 22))
 (segment (start 119.38 67.31) (end 119.38 64.77) (width 0.75) (layer "F.Cu") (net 22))
 (segment (start 110.49 64.77) (end 110.49 58.42) (width 0.75) (layer "F.Cu") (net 22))
 (segment (start 124.46 67.31) (end 124.46 62.23) (width 0.75) (layer "F.Cu") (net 20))
 (segment (start 124.46 62.23) (end 120.65 62.23) (width 0.75) (layer "F.Cu") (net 20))
 (segment (start 120.65 62.23) (end 120.65 58.42) (width 0.75) (layer "F.Cu") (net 20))
 (segment (start 115.57 63.5) (end 115.57 58.42) (width 0.75) (layer "F.Cu") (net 21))
 (segment (start 121.92 63.5) (end 115.57 63.5) (width 0.75) (layer "F.Cu") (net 21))
 (segment (start 121.92 67.31) (end 121.92 63.5) (width 0.75) (layer "F.Cu") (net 21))
 (segment (start 134.62 63.5) (end 140.97 63.5) (width 0.75) (layer "F.Cu") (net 16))
 (segment (start 140.97 63.5) (end 140.97 58.42) (width 0.75) (layer "F.Cu") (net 16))
 (segment (start 134.62 67.31) (end 134.62 63.5) (width 0.75) (layer "F.Cu") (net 16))
 (segment (start 137.16 64.77) (end 146.05 64.77) (width 0.75) (layer "F.Cu") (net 15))
 (segment (start 137.16 67.31) (end 137.16 64.77) (width 0.75) (layer "F.Cu") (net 15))
 (segment (start 146.05 64.77) (end 146.05 58.42) (width 0.75) (layer "F.Cu") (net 15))
 (segment (start 160.02 64.77) (end 151.13 64.77) (width 0.75) (layer "F.Cu") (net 14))
 (segment (start 160.02 67.31) (end 160.02 64.77) (width 0.75) (layer "F.Cu") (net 14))
 (segment (start 151.13 64.77) (end 151.13 58.42) (width 0.75) (layer "F.Cu") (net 14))
 (segment (start 156.21 63.5) (end 156.21 58.42) (width 0.75) (layer "F.Cu") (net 13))
 (segment (start 162.56 67.31) (end 162.56 63.5) (width 0.75) (layer "F.Cu") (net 13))
 (segment (start 162.56 63.5) (end 156.21 63.5) (width 0.75) (layer "F.Cu") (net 13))
 (segment (start 161.29 62.23) (end 161.29 58.42) (width 0.75) (layer "F.Cu") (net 12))
 (segment (start 165.1 67.31) (end 165.1 62.23) (width 0.75) (layer "F.Cu") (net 12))
 (segment (start 165.1 62.23) (end 161.29 62.23) (width 0.75) (layer "F.Cu") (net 12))
 (segment (start 167.64 67.31) (end 167.64 60.96) (width 0.75) (layer "F.Cu") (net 11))
 (segment (start 166.37 60.96) (end 166.37 58.42) (width 0.75) (layer "F.Cu") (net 11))
 (segment (start 167.64 60.96) (end 166.37 60.96) (width 0.75) (layer "F.Cu") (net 11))
 (segment (start 170.18 67.31) (end 170.18 60.96) (width 0.75) (layer "F.Cu") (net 10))
 (segment (start 171.45 60.96) (end 171.45 58.42) (width 0.75) (layer "F.Cu") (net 10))
 (segment (start 170.18 60.96) (end 171.45 60.96) (width 0.75) (layer "F.Cu") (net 10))
 (segment (start 176.53 62.23) (end 176.53 58.42) (width 0.75) (layer "F.Cu") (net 9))
 (segment (start 172.72 62.23) (end 176.53 62.23) (width 0.75) (layer "F.Cu") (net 9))
 (segment (start 172.72 67.31) (end 172.72 62.23) (width 0.75) (layer "F.Cu") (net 9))
 (segment (start 181.61 63.5) (end 181.61 58.42) (width 0.75) (layer "F.Cu") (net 8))
 (segment (start 175.26 63.5) (end 181.61 63.5) (width 0.75) (layer "F.Cu") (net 8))
 (segment (start 175.26 67.31) (end 175.26 63.5) (width 0.75) (layer "F.Cu") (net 8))
 (segment (start 177.8 64.77) (end 186.69 64.77) (width 0.75) (layer "F.Cu") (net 7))
 (segment (start 186.69 64.77) (end 186.69 58.42) (width 0.75) (layer "F.Cu") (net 7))
 (segment (start 177.8 67.31) (end 177.8 64.77) (width 0.75) (layer "F.Cu") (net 7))
 (segment (start 186.69 69.85) (end 180.34 69.85) (width 0.75) (layer "F.Cu") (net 23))
 (segment (start 189.23 67.31) (end 186.69 67.31) (width 0.75) (layer "F.Cu") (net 23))
 (segment (start 180.34 69.85) (end 139.7 69.85) (width 0.75) (layer "F.Cu") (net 23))
 (segment (start 180.34 67.31) (end 180.34 69.85) (width 0.75) (layer "F.Cu") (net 23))
 (segment (start 186.69 67.31) (end 186.69 69.85) (width 0.75) (layer "F.Cu") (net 23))
 (segment (start 139.7 69.85) (end 139.7 67.31) (width 0.75) (layer "F.Cu") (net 23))
 (segment (start 120.65 82.55) (end 121.92 82.55) (width 0.4) (layer "B.Cu") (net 25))
 (segment (start 120.65 88.265) (end 120.65 82.55) (width 0.4) (layer "B.Cu") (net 25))
 (segment (start 121.92 82.55) (end 121.92 74.93) (width 0.4) (layer "B.Cu") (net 25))
 (segment (start 123.19 88.265) (end 123.19 82.55) (width 0.4) (layer "B.Cu") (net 26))
 (segment (start 123.19 82.55) (end 124.46 82.55) (width 0.4) (layer "B.Cu") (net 26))
 (segment (start 124.46 82.55) (end 124.46 74.93) (width 0.4) (layer "B.Cu") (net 26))
 (segment (start 127 82.55) (end 127 74.93) (width 0.4) (layer "B.Cu") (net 27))
 (segment (start 125.73 88.265) (end 125.73 82.55) (width 0.4) (layer "B.Cu") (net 27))
 (segment (start 125.73 82.55) (end 127 82.55) (width 0.4) (layer "B.Cu") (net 27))
 (segment (start 129.54 81.026) (end 129.54 74.93) (width 0.4) (layer "B.Cu") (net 28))
 (segment (start 128.27 82.55) (end 129.54 82.55) (width 0.4) (layer "B.Cu") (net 28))
 (segment (start 128.27 88.265) (end 128.27 82.55) (width 0.4) (layer "B.Cu") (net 28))
 (segment (start 129.54 82.55) (end 129.54 81.026) (width 0.4) (layer "B.Cu") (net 28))
 (segment (start 130.81 82.55) (end 132.08 82.55) (width 0.4) (layer "B.Cu") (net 29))
 (segment (start 132.08 82.55) (end 132.08 74.93) (width 0.4) (layer "B.Cu") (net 29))
 (segment (start 130.81 88.265) (end 130.81 82.55) (width 0.4) (layer "B.Cu") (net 29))
 (segment (start 134.62 82.55) (end 134.62 81.026) (width 0.4) (layer "B.Cu") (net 30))
 (segment (start 133.35 88.265) (end 133.35 82.55) (width 0.4) (layer "B.Cu") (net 30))
 (segment (start 133.35 82.55) (end 134.62 82.55) (width 0.4) (layer "B.Cu") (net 30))
 (segment (start 134.62 81.026) (end 134.62 74.93) (width 0.4) (layer "B.Cu") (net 30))
 (segment (start 135.89 88.265) (end 135.89 82.55) (width 0.4) (layer "B.Cu") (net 31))
 (segment (start 135.89 82.55) (end 137.16 82.55) (width 0.4) (layer "B.Cu") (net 31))
 (segment (start 137.16 82.55) (end 137.16 74.93) (width 0.4) (layer "B.Cu") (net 31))
 (segment (start 158.75 80.645) (end 158.75 82.55) (width 0.4) (layer "F.Cu") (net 40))
 (segment (start 166.37 82.55) (end 166.37 80.645) (width 0.4) (layer "F.Cu") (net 40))
 (segment (start 138.43 80.645) (end 158.75 80.645) (width 0.4) (layer "F.Cu") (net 40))
 (segment (start 158.75 82.55) (end 166.37 82.55) (width 0.4) (layer "F.Cu") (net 40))
 (segment (start 123.19 80.645) (end 123.19 73.152) (width 0.4) (layer "B.Cu") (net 24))
 (segment (start 123.19 73.152) (end 119.38 73.152) (width 0.4) (layer "B.Cu") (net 24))
 (segment (start 119.38 73.152) (end 119.38 74.93) (width 0.4) (layer "B.Cu") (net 24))
 (segment (start 160.02 73.152) (end 160.02 74.93) (width 0.4) (layer "B.Cu") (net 32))
 (segment (start 163.83 80.645) (end 163.83 73.152) (width 0.4) (layer "B.Cu") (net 32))
 (segment (start 163.83 73.152) (end 160.02 73.152) (width 0.4) (layer "B.Cu") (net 32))
 (segment (start 176.53 82.55) (end 177.8 82.55) (width 0.4) (layer "B.Cu") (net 39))
 (segment (start 176.53 88.265) (end 176.53 82.55) (width 0.4) (layer "B.Cu") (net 39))
 (segment (start 177.8 82.55) (end 177.8 74.93) (width 0.4) (layer "B.Cu") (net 39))
 (segment (start 173.99 88.265) (end 173.99 82.55) (width 0.4) (layer "B.Cu") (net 38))
 (segment (start 175.26 80.138998) (end 175.26 74.93) (width 0.4) (layer "B.Cu") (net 38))
 (segment (start 173.99 82.55) (end 175.26 82.55) (width 0.4) (layer "B.Cu") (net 38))
 (segment (start 175.26 82.55) (end 175.26 80.138998) (width 0.4) (layer "B.Cu") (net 38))
 (segment (start 172.72 82.55) (end 172.72 74.93) (width 0.4) (layer "B.Cu") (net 37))
 (segment (start 171.45 88.265) (end 171.45 82.55) (width 0.4) (layer "B.Cu") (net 37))
 (segment (start 171.45 82.55) (end 172.72 82.55) (width 0.4) (layer "B.Cu") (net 37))
 (segment (start 170.18 82.55) (end 170.18 74.93) (width 0.4) (layer "B.Cu") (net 36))
 (segment (start 168.91 88.265) (end 168.91 82.55) (width 0.4) (layer "B.Cu") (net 36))
 (segment (start 168.91 82.55) (end 170.18 82.55) (width 0.4) (layer "B.Cu") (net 36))
 (segment (start 167.64 82.55) (end 167.64 74.93) (width 0.4) (layer "B.Cu") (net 35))
 (segment (start 166.37 88.265) (end 166.37 82.55) (width 0.4) (layer "B.Cu") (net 35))
 (segment (start 166.37 82.55) (end 167.64 82.55) (width 0.4) (layer "B.Cu") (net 35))
 (segment (start 165.1 82.55) (end 165.1 74.93) (width 0.4) (layer "B.Cu") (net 34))
 (segment (start 163.83 82.55) (end 165.1 82.55) (width 0.4) (layer "B.Cu") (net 34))
 (segment (start 163.83 88.265) (end 163.83 82.55) (width 0.4) (layer "B.Cu") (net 34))
 (segment (start 161.29 88.265) (end 161.29 82.55) (width 0.4) (layer "B.Cu") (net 33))
 (segment (start 161.29 82.55) (end 162.56 82.55) (width 0.4) (layer "B.Cu") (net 33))
 (segment (start 162.56 82.55) (end 162.56 74.93) (width 0.4) (layer "B.Cu") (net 33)))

